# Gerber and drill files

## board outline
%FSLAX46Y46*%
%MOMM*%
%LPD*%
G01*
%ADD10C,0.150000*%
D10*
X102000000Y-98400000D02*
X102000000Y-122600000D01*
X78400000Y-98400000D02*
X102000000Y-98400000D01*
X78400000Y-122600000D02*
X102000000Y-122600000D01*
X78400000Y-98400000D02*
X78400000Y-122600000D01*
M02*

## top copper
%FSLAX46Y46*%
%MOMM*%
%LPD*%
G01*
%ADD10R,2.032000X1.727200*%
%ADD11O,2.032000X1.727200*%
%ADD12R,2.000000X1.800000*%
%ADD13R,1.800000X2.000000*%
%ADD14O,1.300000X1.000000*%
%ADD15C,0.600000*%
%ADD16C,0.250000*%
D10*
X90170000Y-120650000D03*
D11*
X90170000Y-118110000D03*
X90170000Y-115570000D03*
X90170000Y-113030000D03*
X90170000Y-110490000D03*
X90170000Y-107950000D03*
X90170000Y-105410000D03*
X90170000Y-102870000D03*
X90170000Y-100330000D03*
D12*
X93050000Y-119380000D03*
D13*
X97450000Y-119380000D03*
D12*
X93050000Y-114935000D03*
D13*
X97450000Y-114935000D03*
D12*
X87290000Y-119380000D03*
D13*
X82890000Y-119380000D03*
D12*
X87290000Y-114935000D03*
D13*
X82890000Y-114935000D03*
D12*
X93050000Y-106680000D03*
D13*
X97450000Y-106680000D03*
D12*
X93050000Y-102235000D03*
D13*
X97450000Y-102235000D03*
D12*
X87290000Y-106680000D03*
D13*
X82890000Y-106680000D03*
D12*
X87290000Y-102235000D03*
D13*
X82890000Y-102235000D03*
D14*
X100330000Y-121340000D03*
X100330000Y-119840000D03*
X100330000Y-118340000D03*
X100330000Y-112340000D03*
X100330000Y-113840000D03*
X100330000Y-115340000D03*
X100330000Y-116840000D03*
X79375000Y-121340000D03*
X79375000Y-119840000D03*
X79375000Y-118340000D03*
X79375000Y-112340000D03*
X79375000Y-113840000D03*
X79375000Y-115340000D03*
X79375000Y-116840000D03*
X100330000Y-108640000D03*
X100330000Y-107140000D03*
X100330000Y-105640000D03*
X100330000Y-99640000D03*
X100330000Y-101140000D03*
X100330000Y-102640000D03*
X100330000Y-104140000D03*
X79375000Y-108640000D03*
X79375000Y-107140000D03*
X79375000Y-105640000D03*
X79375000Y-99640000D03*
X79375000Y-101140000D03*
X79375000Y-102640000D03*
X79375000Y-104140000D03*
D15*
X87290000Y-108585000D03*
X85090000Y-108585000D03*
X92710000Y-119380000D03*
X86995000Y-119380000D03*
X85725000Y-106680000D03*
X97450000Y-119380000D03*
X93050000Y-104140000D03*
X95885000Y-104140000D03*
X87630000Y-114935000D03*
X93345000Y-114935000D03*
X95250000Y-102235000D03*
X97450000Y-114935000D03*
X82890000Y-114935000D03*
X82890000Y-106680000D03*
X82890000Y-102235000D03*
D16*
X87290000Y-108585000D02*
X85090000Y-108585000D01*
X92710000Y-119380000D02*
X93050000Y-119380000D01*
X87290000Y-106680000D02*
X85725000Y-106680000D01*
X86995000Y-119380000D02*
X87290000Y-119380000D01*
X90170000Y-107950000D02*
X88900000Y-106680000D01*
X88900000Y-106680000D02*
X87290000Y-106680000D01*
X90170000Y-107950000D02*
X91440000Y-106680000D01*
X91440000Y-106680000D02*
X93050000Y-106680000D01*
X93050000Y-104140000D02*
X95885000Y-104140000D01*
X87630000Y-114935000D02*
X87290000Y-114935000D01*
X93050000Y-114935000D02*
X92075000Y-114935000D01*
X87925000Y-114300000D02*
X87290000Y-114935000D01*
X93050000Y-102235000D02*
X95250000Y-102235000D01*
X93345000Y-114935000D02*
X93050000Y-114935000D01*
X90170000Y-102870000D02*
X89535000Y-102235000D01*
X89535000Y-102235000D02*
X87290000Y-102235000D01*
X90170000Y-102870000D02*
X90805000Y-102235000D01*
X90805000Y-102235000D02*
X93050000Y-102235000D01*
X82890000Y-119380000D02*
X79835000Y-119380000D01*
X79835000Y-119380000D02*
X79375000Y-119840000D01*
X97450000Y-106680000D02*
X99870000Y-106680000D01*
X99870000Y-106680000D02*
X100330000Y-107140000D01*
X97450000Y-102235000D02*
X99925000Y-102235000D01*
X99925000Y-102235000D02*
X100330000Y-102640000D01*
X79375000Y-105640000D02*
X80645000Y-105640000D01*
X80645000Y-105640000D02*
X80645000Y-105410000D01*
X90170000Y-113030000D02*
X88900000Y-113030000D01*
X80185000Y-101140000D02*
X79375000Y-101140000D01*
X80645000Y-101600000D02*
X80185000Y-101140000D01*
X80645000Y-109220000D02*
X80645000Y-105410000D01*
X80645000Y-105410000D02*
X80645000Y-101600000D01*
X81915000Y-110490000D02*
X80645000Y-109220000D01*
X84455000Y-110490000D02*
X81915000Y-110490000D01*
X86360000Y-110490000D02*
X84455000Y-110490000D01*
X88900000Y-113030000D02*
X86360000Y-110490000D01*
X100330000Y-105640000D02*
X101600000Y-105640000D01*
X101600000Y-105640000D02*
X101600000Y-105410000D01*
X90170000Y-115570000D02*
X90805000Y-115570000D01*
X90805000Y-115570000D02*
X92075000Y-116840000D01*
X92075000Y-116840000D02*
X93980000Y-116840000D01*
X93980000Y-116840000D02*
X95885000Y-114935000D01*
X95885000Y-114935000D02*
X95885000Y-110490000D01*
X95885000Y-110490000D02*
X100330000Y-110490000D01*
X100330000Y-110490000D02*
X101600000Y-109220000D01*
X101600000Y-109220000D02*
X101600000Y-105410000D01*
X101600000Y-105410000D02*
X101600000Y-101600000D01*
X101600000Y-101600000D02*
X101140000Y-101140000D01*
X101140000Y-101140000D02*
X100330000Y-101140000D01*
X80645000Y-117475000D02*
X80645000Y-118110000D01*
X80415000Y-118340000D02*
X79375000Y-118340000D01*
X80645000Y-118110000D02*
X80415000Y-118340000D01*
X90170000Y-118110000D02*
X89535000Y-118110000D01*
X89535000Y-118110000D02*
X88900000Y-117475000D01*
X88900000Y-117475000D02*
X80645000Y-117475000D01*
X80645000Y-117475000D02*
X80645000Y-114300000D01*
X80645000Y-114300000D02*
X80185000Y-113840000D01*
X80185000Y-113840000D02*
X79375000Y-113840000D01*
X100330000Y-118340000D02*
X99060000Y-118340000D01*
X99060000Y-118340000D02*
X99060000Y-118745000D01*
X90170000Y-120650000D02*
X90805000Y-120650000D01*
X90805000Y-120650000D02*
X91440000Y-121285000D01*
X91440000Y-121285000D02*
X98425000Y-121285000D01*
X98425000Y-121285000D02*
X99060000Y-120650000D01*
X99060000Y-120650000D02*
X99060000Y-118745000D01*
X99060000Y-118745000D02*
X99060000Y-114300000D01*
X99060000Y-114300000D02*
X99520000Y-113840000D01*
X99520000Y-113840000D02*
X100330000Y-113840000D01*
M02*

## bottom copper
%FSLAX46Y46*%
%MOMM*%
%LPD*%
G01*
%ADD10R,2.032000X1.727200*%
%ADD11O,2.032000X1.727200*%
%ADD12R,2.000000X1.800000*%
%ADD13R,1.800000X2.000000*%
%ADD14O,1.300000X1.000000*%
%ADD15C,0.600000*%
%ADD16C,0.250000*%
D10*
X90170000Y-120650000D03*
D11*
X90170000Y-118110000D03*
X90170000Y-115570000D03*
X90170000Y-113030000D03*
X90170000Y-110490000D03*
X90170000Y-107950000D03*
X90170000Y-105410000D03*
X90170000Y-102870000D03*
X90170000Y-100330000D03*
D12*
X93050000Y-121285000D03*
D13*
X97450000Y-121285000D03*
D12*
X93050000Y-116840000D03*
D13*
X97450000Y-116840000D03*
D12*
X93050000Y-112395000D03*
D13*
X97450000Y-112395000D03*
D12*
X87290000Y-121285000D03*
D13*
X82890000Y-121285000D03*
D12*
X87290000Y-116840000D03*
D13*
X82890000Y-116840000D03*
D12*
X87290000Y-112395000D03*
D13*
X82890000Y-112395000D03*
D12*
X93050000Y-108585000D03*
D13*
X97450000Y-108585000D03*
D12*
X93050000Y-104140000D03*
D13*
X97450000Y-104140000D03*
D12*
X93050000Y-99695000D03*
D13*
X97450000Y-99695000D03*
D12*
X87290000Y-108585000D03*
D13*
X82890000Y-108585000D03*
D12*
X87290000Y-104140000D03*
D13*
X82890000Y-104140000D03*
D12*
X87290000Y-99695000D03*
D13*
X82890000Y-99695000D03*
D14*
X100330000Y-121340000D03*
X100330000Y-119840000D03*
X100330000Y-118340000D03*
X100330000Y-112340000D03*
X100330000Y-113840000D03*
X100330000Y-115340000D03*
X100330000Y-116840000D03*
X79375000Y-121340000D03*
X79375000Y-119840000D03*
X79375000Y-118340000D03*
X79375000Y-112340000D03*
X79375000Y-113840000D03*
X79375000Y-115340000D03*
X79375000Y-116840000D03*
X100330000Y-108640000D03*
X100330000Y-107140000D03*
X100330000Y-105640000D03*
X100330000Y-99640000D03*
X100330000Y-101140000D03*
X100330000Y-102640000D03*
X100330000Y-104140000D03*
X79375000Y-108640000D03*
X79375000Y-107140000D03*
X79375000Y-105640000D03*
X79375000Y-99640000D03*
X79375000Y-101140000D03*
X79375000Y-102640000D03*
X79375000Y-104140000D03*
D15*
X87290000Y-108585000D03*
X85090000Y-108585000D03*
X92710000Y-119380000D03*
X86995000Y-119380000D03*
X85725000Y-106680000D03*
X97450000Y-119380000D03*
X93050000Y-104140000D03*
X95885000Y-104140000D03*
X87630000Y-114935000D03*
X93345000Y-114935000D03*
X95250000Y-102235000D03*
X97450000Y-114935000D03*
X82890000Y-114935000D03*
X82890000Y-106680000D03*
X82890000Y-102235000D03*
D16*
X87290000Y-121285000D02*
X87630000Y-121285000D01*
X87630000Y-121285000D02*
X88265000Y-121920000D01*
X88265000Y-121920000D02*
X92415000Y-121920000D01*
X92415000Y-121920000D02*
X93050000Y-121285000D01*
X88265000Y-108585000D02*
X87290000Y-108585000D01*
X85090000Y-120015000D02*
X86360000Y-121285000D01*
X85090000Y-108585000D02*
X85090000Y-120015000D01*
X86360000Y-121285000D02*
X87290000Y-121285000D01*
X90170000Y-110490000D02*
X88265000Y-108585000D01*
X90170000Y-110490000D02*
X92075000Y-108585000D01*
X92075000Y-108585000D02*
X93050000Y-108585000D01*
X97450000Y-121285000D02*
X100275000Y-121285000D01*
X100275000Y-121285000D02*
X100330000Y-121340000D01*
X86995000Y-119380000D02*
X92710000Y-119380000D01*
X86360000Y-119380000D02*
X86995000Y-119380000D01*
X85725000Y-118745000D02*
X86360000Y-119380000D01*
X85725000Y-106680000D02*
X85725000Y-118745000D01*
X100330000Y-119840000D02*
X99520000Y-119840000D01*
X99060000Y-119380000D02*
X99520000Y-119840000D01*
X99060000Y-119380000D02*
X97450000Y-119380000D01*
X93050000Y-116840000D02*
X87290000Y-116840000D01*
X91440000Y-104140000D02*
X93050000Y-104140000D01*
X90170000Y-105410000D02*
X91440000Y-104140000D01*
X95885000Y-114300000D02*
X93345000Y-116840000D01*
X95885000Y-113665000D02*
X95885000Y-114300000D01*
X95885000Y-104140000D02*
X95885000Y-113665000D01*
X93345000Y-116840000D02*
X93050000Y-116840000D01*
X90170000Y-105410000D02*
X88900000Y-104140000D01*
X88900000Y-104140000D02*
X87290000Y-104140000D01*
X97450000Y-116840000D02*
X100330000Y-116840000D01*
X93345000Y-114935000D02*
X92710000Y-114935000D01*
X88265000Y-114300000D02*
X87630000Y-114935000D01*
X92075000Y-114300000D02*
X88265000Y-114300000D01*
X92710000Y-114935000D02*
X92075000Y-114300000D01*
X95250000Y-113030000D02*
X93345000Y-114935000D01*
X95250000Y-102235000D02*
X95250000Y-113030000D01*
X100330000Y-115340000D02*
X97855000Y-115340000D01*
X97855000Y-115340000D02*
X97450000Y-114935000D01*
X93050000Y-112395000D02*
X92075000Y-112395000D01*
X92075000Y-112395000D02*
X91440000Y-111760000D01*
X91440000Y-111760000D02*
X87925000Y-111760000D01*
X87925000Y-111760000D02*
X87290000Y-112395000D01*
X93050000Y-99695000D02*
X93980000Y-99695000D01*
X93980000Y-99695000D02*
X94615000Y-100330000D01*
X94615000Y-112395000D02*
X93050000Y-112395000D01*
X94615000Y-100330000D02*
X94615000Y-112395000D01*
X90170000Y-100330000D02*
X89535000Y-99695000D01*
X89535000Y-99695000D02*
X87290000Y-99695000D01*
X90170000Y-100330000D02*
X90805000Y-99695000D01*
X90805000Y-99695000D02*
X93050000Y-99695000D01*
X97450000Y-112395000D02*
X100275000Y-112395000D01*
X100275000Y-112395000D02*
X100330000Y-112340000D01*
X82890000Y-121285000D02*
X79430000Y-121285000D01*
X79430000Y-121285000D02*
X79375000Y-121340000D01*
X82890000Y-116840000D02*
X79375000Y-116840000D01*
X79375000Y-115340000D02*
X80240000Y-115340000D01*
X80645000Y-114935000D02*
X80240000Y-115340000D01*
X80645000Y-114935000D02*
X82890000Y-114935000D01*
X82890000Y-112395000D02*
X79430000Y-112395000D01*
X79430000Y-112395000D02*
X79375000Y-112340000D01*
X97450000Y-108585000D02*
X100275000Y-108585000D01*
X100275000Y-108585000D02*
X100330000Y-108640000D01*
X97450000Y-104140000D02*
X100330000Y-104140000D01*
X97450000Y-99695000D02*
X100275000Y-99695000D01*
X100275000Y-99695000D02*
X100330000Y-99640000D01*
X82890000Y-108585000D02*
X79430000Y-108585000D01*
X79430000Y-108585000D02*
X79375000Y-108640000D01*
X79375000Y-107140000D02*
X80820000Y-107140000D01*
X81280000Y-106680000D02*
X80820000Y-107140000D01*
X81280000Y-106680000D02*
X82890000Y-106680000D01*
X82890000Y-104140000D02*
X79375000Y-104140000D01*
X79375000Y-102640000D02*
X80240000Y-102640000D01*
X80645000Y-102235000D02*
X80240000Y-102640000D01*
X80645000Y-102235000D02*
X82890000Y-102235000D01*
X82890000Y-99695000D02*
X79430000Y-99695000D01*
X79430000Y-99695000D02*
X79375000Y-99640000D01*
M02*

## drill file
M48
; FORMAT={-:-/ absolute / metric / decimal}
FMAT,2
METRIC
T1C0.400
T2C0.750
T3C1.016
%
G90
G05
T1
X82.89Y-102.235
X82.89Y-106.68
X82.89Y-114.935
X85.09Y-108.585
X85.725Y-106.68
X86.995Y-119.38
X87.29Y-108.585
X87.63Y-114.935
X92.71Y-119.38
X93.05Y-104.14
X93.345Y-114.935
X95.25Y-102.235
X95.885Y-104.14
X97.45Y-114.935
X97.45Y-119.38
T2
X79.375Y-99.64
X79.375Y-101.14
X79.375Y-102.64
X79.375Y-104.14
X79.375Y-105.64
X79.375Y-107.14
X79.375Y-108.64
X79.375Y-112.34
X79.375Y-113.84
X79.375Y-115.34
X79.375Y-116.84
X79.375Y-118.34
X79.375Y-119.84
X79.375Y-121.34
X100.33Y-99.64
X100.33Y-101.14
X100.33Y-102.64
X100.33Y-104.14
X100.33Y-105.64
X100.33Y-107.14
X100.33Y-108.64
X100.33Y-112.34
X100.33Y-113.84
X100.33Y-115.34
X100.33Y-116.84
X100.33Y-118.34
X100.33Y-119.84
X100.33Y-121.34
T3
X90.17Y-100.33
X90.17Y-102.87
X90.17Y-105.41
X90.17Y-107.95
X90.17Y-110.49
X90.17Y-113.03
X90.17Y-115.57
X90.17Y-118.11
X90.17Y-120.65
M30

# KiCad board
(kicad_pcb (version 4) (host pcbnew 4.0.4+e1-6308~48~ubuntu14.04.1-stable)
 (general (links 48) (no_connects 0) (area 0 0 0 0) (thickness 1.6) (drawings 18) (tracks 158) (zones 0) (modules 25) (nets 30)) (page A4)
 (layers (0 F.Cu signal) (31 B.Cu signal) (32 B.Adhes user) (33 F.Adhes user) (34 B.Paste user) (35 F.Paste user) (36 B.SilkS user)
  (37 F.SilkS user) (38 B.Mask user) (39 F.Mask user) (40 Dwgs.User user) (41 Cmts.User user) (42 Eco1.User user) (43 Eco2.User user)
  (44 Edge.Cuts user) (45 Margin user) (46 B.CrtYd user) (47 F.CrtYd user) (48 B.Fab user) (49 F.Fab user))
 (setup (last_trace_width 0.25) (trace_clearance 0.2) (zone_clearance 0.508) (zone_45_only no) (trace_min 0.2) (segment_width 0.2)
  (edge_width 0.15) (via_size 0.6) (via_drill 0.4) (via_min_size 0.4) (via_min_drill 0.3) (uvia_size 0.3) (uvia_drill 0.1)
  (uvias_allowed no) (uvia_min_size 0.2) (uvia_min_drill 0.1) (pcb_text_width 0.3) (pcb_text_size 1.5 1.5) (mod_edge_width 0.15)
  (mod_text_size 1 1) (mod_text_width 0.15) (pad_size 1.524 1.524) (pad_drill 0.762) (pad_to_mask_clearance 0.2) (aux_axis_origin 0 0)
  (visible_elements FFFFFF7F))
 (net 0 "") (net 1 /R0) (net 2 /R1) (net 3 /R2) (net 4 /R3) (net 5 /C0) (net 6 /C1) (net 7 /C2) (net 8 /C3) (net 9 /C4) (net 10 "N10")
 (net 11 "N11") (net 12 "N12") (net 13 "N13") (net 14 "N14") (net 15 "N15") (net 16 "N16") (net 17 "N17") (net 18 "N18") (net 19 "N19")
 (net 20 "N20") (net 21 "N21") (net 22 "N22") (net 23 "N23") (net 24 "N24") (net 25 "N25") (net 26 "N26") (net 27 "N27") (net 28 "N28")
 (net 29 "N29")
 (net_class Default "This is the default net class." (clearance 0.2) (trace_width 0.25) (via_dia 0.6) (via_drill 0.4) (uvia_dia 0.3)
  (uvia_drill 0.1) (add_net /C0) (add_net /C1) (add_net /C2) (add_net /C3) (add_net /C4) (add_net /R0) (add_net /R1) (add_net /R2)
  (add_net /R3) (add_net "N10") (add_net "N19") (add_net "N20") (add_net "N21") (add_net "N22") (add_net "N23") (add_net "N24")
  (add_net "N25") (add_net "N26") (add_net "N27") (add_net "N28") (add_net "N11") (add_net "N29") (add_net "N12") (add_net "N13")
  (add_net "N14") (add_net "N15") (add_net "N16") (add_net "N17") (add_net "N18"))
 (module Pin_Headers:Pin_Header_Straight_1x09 (layer B.Cu) (at 90.17 120.65)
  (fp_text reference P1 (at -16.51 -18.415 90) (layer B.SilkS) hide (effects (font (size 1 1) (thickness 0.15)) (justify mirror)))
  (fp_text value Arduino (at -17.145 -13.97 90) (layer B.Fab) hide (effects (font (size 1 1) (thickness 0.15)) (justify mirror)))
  (pad 1 thru_hole rect (at 0 0) (size 2.032 1.7272) (drill 1.016) (layers *.Cu *.Mask B.SilkS) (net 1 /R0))
  (pad 2 thru_hole oval (at 0 -2.54) (size 2.032 1.7272) (drill 1.016) (layers *.Cu *.Mask B.SilkS) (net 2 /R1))
  (pad 3 thru_hole oval (at 0 -5.08) (size 2.032 1.7272) (drill 1.016) (layers *.Cu *.Mask B.SilkS) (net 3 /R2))
  (pad 4 thru_hole oval (at 0 -7.62) (size 2.032 1.7272) (drill 1.016) (layers *.Cu *.Mask B.SilkS) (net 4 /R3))
  (pad 5 thru_hole oval (at 0 -10.16) (size 2.032 1.7272) (drill 1.016) (layers *.Cu *.Mask B.SilkS) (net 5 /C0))
  (pad 6 thru_hole oval (at 0 -12.7) (size 2.032 1.7272) (drill 1.016) (layers *.Cu *.Mask B.SilkS) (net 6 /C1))
  (pad 7 thru_hole oval (at 0 -15.24) (size 2.032 1.7272) (drill 1.016) (layers *.Cu *.Mask B.SilkS) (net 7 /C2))
  (pad 8 thru_hole oval (at 0 -17.78) (size 2.032 1.7272) (drill 1.016) (layers *.Cu *.Mask B.SilkS) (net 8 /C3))
  (pad 9 thru_hole oval (at 0 -20.32) (size 2.032 1.7272) (drill 1.016) (layers *.Cu *.Mask B.SilkS) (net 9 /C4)))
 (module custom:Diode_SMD (layer B.Cu) (at 95.25 121.285 180)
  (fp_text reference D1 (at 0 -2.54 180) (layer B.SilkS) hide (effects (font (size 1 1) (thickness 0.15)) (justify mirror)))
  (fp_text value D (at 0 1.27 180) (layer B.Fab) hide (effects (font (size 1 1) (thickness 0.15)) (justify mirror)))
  (pad 2 smd rect (at 2.2 0 180) (size 2 1.8) (layers B.Cu B.Paste B.Mask) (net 5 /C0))
  (pad 1 smd rect (at -2.2 0 180) (size 1.8 2) (layers B.Cu B.Paste B.Mask) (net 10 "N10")))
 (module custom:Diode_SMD (layer F.Cu) (at 95.25 119.38 180)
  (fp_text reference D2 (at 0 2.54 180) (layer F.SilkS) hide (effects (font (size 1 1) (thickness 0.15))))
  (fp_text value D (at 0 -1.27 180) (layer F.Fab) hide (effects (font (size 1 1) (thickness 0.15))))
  (pad 2 smd rect (at 2.2 0 180) (size 2 1.8) (layers F.Cu F.Paste F.Mask) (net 6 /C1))
  (pad 1 smd rect (at -2.2 0 180) (size 1.8 2) (layers F.Cu F.Paste F.Mask) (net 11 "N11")))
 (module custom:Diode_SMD (layer B.Cu) (at 95.25 116.84 180)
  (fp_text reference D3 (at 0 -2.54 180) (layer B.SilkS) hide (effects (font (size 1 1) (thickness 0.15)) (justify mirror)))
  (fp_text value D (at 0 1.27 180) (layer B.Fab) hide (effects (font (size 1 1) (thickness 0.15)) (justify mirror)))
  (pad 2 smd rect (at 2.2 0 180) (size 2 1.8) (layers B.Cu B.Paste B.Mask) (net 7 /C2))
  (pad 1 smd rect (at -2.2 0 180) (size 1.8 2) (layers B.Cu B.Paste B.Mask) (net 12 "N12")))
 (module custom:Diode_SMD (layer F.Cu) (at 95.25 114.935 180)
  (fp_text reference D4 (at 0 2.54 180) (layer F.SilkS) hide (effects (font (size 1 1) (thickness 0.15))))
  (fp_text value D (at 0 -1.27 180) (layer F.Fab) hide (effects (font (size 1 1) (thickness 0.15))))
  (pad 2 smd rect (at 2.2 0 180) (size 2 1.8) (layers F.Cu F.Paste F.Mask) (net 8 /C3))
  (pad 1 smd rect (at -2.2 0 180) (size 1.8 2) (layers F.Cu F.Paste F.Mask) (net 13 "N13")))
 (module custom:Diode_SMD (layer B.Cu) (at 95.25 112.395 180)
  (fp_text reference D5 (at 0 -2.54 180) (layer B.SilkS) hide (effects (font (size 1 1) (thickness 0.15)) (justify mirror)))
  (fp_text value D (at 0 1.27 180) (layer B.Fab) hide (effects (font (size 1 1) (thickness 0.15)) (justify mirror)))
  (pad 2 smd rect (at 2.2 0 180) (size 2 1.8) (layers B.Cu B.Paste B.Mask) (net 9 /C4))
  (pad 1 smd rect (at -2.2 0 180) (size 1.8 2) (layers B.Cu B.Paste B.Mask) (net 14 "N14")))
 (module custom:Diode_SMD (layer B.Cu) (at 85.09 121.285)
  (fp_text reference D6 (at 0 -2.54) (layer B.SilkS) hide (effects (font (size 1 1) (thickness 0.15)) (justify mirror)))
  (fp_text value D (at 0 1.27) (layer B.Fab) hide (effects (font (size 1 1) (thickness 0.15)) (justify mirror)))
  (pad 2 smd rect (at 2.2 0) (size 2 1.8) (layers B.Cu B.Paste B.Mask) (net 5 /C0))
  (pad 1 smd rect (at -2.2 0) (size 1.8 2) (layers B.Cu B.Paste B.Mask) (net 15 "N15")))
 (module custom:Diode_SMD (layer F.Cu) (at 85.09 119.38)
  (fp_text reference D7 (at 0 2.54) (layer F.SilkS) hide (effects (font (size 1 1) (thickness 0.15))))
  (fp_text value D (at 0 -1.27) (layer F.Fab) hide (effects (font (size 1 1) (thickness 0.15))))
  (pad 2 smd rect (at 2.2 0) (size 2 1.8) (layers F.Cu F.Paste F.Mask) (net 6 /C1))
  (pad 1 smd rect (at -2.2 0) (size 1.8 2) (layers F.Cu F.Paste F.Mask) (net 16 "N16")))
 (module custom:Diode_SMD (layer B.Cu) (at 85.09 116.84)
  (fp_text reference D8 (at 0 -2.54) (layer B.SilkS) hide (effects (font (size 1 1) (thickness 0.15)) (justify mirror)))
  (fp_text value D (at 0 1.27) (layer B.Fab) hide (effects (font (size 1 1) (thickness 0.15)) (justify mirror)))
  (pad 2 smd rect (at 2.2 0) (size 2 1.8) (layers B.Cu B.Paste B.Mask) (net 7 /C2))
  (pad 1 smd rect (at -2.2 0) (size 1.8 2) (layers B.Cu B.Paste B.Mask) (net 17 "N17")))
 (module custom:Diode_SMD (layer F.Cu) (at 85.09 114.935)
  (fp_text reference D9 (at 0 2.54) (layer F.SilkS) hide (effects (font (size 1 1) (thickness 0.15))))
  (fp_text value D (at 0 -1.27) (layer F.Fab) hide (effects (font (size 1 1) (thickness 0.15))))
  (pad 2 smd rect (at 2.2 0) (size 2 1.8) (layers F.Cu F.Paste F.Mask) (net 8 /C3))
  (pad 1 smd rect (at -2.2 0) (size 1.8 2) (layers F.Cu F.Paste F.Mask) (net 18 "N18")))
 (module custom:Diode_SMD (layer B.Cu) (at 85.09 112.395)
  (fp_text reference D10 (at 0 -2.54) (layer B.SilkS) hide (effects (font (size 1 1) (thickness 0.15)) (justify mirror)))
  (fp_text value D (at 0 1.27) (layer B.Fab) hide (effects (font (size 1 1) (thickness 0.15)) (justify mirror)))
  (pad 2 smd rect (at 2.2 0) (size 2 1.8) (layers B.Cu B.Paste B.Mask) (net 9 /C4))
  (pad 1 smd rect (at -2.2 0) (size 1.8 2) (layers B.Cu B.Paste B.Mask) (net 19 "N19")))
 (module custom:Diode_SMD (layer B.Cu) (at 95.25 108.585 180)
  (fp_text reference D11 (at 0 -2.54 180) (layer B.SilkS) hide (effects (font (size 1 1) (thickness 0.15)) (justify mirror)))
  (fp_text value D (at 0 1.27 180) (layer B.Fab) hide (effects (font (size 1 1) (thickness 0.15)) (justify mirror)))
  (pad 2 smd rect (at 2.2 0 180) (size 2 1.8) (layers B.Cu B.Paste B.Mask) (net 5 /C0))
  (pad 1 smd rect (at -2.2 0 180) (size 1.8 2) (layers B.Cu B.Paste B.Mask) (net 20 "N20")))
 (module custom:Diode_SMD (layer F.Cu) (at 95.25 106.68 180)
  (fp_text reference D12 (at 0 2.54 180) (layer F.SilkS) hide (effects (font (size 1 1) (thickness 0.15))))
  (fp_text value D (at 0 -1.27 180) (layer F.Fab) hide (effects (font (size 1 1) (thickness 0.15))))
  (pad 2 smd rect (at 2.2 0 180) (size 2 1.8) (layers F.Cu F.Paste F.Mask) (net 6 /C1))
  (pad 1 smd rect (at -2.2 0 180) (size 1.8 2) (layers F.Cu F.Paste F.Mask) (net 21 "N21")))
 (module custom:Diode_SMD (layer B.Cu) (at 95.25 104.14 180)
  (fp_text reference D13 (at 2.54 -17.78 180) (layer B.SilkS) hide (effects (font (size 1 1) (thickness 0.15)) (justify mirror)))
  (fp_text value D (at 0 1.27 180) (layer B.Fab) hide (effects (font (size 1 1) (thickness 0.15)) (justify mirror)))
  (pad 2 smd rect (at 2.2 0 180) (size 2 1.8) (layers B.Cu B.Paste B.Mask) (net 7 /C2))
  (pad 1 smd rect (at -2.2 0 180) (size 1.8 2) (layers B.Cu B.Paste B.Mask) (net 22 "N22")))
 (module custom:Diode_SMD (layer F.Cu) (at 95.25 102.235 180)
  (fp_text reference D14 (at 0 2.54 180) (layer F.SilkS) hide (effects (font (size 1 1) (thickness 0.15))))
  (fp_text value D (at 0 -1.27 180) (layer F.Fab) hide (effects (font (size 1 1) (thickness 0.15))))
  (pad 2 smd rect (at 2.2 0 180) (size 2 1.8) (layers F.Cu F.Paste F.Mask) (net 8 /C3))
  (pad 1 smd rect (at -2.2 0 180) (size 1.8 2) (layers F.Cu F.Paste F.Mask) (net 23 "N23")))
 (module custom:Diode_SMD (layer B.Cu) (at 95.25 99.695 180)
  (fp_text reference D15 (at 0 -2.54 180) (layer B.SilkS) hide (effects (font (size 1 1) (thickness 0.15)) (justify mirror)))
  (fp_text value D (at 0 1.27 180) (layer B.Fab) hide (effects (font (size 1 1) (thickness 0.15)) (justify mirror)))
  (pad 2 smd rect (at 2.2 0 180) (size 2 1.8) (layers B.Cu B.Paste B.Mask) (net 9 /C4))
  (pad 1 smd rect (at -2.2 0 180) (size 1.8 2) (layers B.Cu B.Paste B.Mask) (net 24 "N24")))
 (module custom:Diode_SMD (layer B.Cu) (at 85.09 108.585)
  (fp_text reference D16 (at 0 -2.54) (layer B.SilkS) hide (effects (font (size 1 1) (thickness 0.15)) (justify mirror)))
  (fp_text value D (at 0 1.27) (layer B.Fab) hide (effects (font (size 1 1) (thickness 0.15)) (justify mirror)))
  (pad 2 smd rect (at 2.2 0) (size 2 1.8) (layers B.Cu B.Paste B.Mask) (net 5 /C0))
  (pad 1 smd rect (at -2.2 0) (size 1.8 2) (layers B.Cu B.Paste B.Mask) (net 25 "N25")))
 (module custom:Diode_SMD (layer F.Cu) (at 85.09 106.68)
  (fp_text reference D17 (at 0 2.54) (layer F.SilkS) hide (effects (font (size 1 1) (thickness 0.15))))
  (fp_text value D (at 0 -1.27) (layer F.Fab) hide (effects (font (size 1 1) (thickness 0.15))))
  (pad 2 smd rect (at 2.2 0) (size 2 1.8) (layers F.Cu F.Paste F.Mask) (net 6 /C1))
  (pad 1 smd rect (at -2.2 0) (size 1.8 2) (layers F.Cu F.Paste F.Mask) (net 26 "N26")))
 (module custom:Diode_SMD (layer B.Cu) (at 85.09 104.14)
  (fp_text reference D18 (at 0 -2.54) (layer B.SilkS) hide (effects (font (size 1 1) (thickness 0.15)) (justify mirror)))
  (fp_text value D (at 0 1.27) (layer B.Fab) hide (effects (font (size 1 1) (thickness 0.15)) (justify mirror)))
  (pad 2 smd rect (at 2.2 0) (size 2 1.8) (layers B.Cu B.Paste B.Mask) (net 7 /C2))
  (pad 1 smd rect (at -2.2 0) (size 1.8 2) (layers B.Cu B.Paste B.Mask) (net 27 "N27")))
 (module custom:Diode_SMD (layer F.Cu) (at 85.09 102.235)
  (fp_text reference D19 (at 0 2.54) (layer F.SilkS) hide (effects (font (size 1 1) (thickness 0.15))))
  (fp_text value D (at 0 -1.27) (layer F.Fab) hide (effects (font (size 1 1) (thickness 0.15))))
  (pad 2 smd rect (at 2.2 0) (size 2 1.8) (layers F.Cu F.Paste F.Mask) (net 8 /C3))
  (pad 1 smd rect (at -2.2 0) (size 1.8 2) (layers F.Cu F.Paste F.Mask) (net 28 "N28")))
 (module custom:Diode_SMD (layer B.Cu) (at 85.09 99.695)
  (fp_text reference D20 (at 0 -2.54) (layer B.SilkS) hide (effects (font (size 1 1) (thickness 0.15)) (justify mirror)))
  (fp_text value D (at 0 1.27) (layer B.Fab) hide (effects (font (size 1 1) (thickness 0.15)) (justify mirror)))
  (pad 2 smd rect (at 2.2 0) (size 2 1.8) (layers B.Cu B.Paste B.Mask) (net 9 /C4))
  (pad 1 smd rect (at -2.2 0) (size 1.8 2) (layers B.Cu B.Paste B.Mask) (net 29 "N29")))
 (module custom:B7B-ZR (layer F.Cu) (at 100.33 116.84 90)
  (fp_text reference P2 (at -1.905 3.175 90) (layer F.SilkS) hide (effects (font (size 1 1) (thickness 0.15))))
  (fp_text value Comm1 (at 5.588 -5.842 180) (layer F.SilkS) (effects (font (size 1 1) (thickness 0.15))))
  (pad 1 thru_hole oval (at -4.5 0 90) (size 1 1.3) (drill 0.75) (layers *.Cu *.Mask F.Paste) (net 10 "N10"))
  (pad 2 thru_hole oval (at -3 0 90) (size 1 1.3) (drill 0.75) (layers *.Cu *.Mask F.Paste) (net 11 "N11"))
  (pad 3 thru_hole oval (at -1.5 0 90) (size 1 1.3) (drill 0.75) (layers *.Cu *.Mask F.Paste) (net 1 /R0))
  (pad 7 thru_hole oval (at 4.5 0 90) (size 1 1.3) (drill 0.75) (layers *.Cu *.Mask F.Paste) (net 14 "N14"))
  (pad 6 thru_hole oval (at 3 0 90) (size 1 1.3) (drill 0.75) (layers *.Cu *.Mask F.Paste) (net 1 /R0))
  (pad 5 thru_hole oval (at 1.5 0 90) (size 1 1.3) (drill 0.75) (layers *.Cu *.Mask F.Paste) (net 13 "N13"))
  (pad 4 thru_hole oval (at 0 0 90) (size 1 1.3) (drill 0.75) (layers *.Cu *.Mask F.Paste) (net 12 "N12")))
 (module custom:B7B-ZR (layer F.Cu) (at 79.375 116.84 90)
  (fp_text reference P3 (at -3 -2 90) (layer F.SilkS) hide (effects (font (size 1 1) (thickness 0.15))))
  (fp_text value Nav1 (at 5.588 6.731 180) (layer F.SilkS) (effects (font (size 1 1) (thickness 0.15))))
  (pad 1 thru_hole oval (at -4.5 0 90) (size 1 1.3) (drill 0.75) (layers *.Cu *.Mask F.Paste) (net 15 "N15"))
  (pad 2 thru_hole oval (at -3 0 90) (size 1 1.3) (drill 0.75) (layers *.Cu *.Mask F.Paste) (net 16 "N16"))
  (pad 3 thru_hole oval (at -1.5 0 90) (size 1 1.3) (drill 0.75) (layers *.Cu *.Mask F.Paste) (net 2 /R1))
  (pad 7 thru_hole oval (at 4.5 0 90) (size 1 1.3) (drill 0.75) (layers *.Cu *.Mask F.Paste) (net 19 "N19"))
  (pad 6 thru_hole oval (at 3 0 90) (size 1 1.3) (drill 0.75) (layers *.Cu *.Mask F.Paste) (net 2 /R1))
  (pad 5 thru_hole oval (at 1.5 0 90) (size 1 1.3) (drill 0.75) (layers *.Cu *.Mask F.Paste) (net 18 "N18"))
  (pad 4 thru_hole oval (at 0 0 90) (size 1 1.3) (drill 0.75) (layers *.Cu *.Mask F.Paste) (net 17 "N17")))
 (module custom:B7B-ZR (layer F.Cu) (at 100.33 104.14 90)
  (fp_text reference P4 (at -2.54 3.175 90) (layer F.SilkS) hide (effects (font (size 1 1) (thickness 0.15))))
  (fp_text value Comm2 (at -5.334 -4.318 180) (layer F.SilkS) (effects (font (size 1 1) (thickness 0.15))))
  (pad 1 thru_hole oval (at -4.5 0 90) (size 1 1.3) (drill 0.75) (layers *.Cu *.Mask F.Paste) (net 20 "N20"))
  (pad 2 thru_hole oval (at -3 0 90) (size 1 1.3) (drill 0.75) (layers *.Cu *.Mask F.Paste) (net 21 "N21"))
  (pad 3 thru_hole oval (at -1.5 0 90) (size 1 1.3) (drill 0.75) (layers *.Cu *.Mask F.Paste) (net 3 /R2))
  (pad 7 thru_hole oval (at 4.5 0 90) (size 1 1.3) (drill 0.75) (layers *.Cu *.Mask F.Paste) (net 24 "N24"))
  (pad 6 thru_hole oval (at 3 0 90) (size 1 1.3) (drill 0.75) (layers *.Cu *.Mask F.Paste) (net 3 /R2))
  (pad 5 thru_hole oval (at 1.5 0 90) (size 1 1.3) (drill 0.75) (layers *.Cu *.Mask F.Paste) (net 23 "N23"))
  (pad 4 thru_hole oval (at 0 0 90) (size 1 1.3) (drill 0.75) (layers *.Cu *.Mask F.Paste) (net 22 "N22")))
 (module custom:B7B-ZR (layer F.Cu) (at 79.375 104.14 90)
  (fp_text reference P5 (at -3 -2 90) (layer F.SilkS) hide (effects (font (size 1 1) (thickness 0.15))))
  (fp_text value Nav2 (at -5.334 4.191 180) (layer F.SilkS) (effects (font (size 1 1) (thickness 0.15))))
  (pad 1 thru_hole oval (at -4.5 0 90) (size 1 1.3) (drill 0.75) (layers *.Cu *.Mask F.Paste) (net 25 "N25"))
  (pad 2 thru_hole oval (at -3 0 90) (size 1 1.3) (drill 0.75) (layers *.Cu *.Mask F.Paste) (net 26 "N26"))
  (pad 3 thru_hole oval (at -1.5 0 90) (size 1 1.3) (drill 0.75) (layers *.Cu *.Mask F.Paste) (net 4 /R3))
  (pad 7 thru_hole oval (at 4.5 0 90) (size 1 1.3) (drill 0.75) (layers *.Cu *.Mask F.Paste) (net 29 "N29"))
  (pad 6 thru_hole oval (at 3 0 90) (size 1 1.3) (drill 0.75) (layers *.Cu *.Mask F.Paste) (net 4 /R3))
  (pad 5 thru_hole oval (at 1.5 0 90) (size 1 1.3) (drill 0.75) (layers *.Cu *.Mask F.Paste) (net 28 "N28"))
  (pad 4 thru_hole oval (at 0 0 90) (size 1 1.3) (drill 0.75) (layers *.Cu *.Mask F.Paste) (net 27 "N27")))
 (gr_line (start 102 98.4) (end 102 122.6) (angle 90) (layer Edge.Cuts) (width 0.15))
 (gr_line (start 78.4 98.4) (end 102 98.4) (angle 90) (layer Edge.Cuts) (width 0.15))
 (gr_line (start 78.4 122.6) (end 102 122.6) (angle 90) (layer Edge.Cuts) (width 0.15))
 (gr_line (start 78.4 98.4) (end 78.4 122.6) (angle 90) (layer Edge.Cuts) (width 0.15))
 (segment (start 87.29 121.285) (end 87.63 121.285) (width 0.25) (layer B.Cu) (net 5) (status C00000))
 (segment (start 87.63 121.285) (end 88.265 121.92) (width 0.25) (layer B.Cu) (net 5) (status C00000))
 (segment (start 88.265 121.92) (end 92.415 121.92) (width 0.25) (layer B.Cu) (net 5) (status C00000))
 (segment (start 92.415 121.92) (end 93.05 121.285) (width 0.25) (layer B.Cu) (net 5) (status C00000))
 (via (at 87.29 108.585) (size 0.6) (drill 0.4) (layers F.Cu B.Cu) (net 5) (status 400000))
 (segment (start 88.265 108.585) (end 87.29 108.585) (width 0.25) (layer B.Cu) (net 5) (status C00000))
 (segment (start 85.09 120.015) (end 86.36 121.285) (width 0.25) (layer B.Cu) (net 5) (status 800000))
 (segment (start 85.09 108.585) (end 85.09 120.015) (width 0.25) (layer B.Cu) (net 5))
 (via (at 85.09 108.585) (size 0.6) (drill 0.4) (layers F.Cu B.Cu) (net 5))
 (segment (start 87.29 108.585) (end 85.09 108.585) (width 0.25) (layer F.Cu) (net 5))
 (segment (start 86.36 121.285) (end 87.29 121.285) (width 0.25) (layer B.Cu) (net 5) (status C00000))
 (segment (start 90.17 110.49) (end 88.265 108.585) (width 0.25) (layer B.Cu) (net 5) (status C00000))
 (segment (start 90.17 110.49) (end 92.075 108.585) (width 0.25) (layer B.Cu) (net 5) (status C00000))
 (segment (start 92.075 108.585) (end 93.05 108.585) (width 0.25) (layer B.Cu) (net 5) (status C00000))
 (segment (start 97.45 121.285) (end 100.275 121.285) (width 0.25) (layer B.Cu) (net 10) (status C00000))
 (segment (start 100.275 121.285) (end 100.33 121.34) (width 0.25) (layer B.Cu) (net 10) (status C00000))
 (segment (start 86.995 119.38) (end 92.71 119.38) (width 0.25) (layer B.Cu) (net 6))
 (segment (start 92.71 119.38) (end 93.05 119.38) (width 0.25) (layer F.Cu) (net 6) (status C00000))
 (via (at 92.71 119.38) (size 0.6) (drill 0.4) (layers F.Cu B.Cu) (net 6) (status 800000))
 (segment (start 87.29 106.68) (end 85.725 106.68) (width 0.25) (layer F.Cu) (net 6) (status 400000))
 (segment (start 86.995 119.38) (end 87.29 119.38) (width 0.25) (layer F.Cu) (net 6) (status C00000))
 (via (at 86.995 119.38) (size 0.6) (drill 0.4) (layers F.Cu B.Cu) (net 6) (status 800000))
 (segment (start 86.36 119.38) (end 86.995 119.38) (width 0.25) (layer B.Cu) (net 6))
 (segment (start 85.725 118.745) (end 86.36 119.38) (width 0.25) (layer B.Cu) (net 6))
 (segment (start 85.725 106.68) (end 85.725 118.745) (width 0.25) (layer B.Cu) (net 6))
 (via (at 85.725 106.68) (size 0.6) (drill 0.4) (layers F.Cu B.Cu) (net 6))
 (segment (start 90.17 107.95) (end 88.9 106.68) (width 0.25) (layer F.Cu) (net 6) (status 400000))
 (segment (start 88.9 106.68) (end 87.29 106.68) (width 0.25) (layer F.Cu) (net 6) (status 800000))
 (segment (start 90.17 107.95) (end 91.44 106.68) (width 0.25) (layer F.Cu) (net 6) (status 400000))
 (segment (start 91.44 106.68) (end 93.05 106.68) (width 0.25) (layer F.Cu) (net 6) (status 800000))
 (via (at 97.45 119.38) (size 0.6) (drill 0.4) (layers F.Cu B.Cu) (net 11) (status C00000))
 (segment (start 100.33 119.84) (end 99.52 119.84) (width 0.25) (layer B.Cu) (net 11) (status 400000))
 (segment (start 99.06 119.38) (end 99.52 119.84) (width 0.25) (layer B.Cu) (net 11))
 (segment (start 99.06 119.38) (end 97.45 119.38) (width 0.25) (layer B.Cu) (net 11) (status 800000))
 (segment (start 93.05 116.84) (end 87.29 116.84) (width 0.25) (layer B.Cu) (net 7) (status C00000))
 (via (at 93.05 104.14) (size 0.6) (drill 0.4) (layers F.Cu B.Cu) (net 7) (status 400000))
 (segment (start 91.44 104.14) (end 93.05 104.14) (width 0.25) (layer B.Cu) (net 7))
 (segment (start 90.17 105.41) (end 91.44 104.14) (width 0.25) (layer B.Cu) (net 7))
 (segment (start 95.885 114.3) (end 93.345 116.84) (width 0.25) (layer B.Cu) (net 7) (status 800000))
 (segment (start 95.885 113.665) (end 95.885 114.3) (width 0.25) (layer B.Cu) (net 7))
 (segment (start 95.885 104.14) (end 95.885 113.665) (width 0.25) (layer B.Cu) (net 7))
 (via (at 95.885 104.14) (size 0.6) (drill 0.4) (layers F.Cu B.Cu) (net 7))
 (segment (start 93.05 104.14) (end 95.885 104.14) (width 0.25) (layer F.Cu) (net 7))
 (segment (start 93.345 116.84) (end 93.05 116.84) (width 0.25) (layer B.Cu) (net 7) (status C00000))
 (segment (start 90.17 105.41) (end 88.9 104.14) (width 0.25) (layer B.Cu) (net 7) (status 400000))
 (segment (start 88.9 104.14) (end 87.29 104.14) (width 0.25) (layer B.Cu) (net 7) (status 800000))
 (segment (start 97.45 116.84) (end 100.33 116.84) (width 0.25) (layer B.Cu) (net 12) (status C00000))
 (segment (start 93.345 114.935) (end 92.71 114.935) (width 0.25) (layer B.Cu) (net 8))
 (segment (start 87.63 114.935) (end 87.29 114.935) (width 0.25) (layer F.Cu) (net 8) (status C00000))
 (via (at 87.63 114.935) (size 0.6) (drill 0.4) (layers F.Cu B.Cu) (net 8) (status 800000))
 (segment (start 88.265 114.3) (end 87.63 114.935) (width 0.25) (layer B.Cu) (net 8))
 (segment (start 92.075 114.3) (end 88.265 114.3) (width 0.25) (layer B.Cu) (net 8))
 (segment (start 92.71 114.935) (end 92.075 114.3) (width 0.25) (layer B.Cu) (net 8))
 (segment (start 93.05 114.935) (end 92.075 114.935) (width 0.25) (layer F.Cu) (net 8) (status C00000))
 (segment (start 87.925 114.3) (end 87.29 114.935) (width 0.25) (layer F.Cu) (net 8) (status C00000))
 (segment (start 93.05 102.235) (end 95.25 102.235) (width 0.25) (layer F.Cu) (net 8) (status 400000))
 (segment (start 93.345 114.935) (end 93.05 114.935) (width 0.25) (layer F.Cu) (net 8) (status C00000))
 (via (at 93.345 114.935) (size 0.6) (drill 0.4) (layers F.Cu B.Cu) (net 8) (status 800000))
 (segment (start 95.25 113.03) (end 93.345 114.935) (width 0.25) (layer B.Cu) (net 8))
 (segment (start 95.25 102.235) (end 95.25 113.03) (width 0.25) (layer B.Cu) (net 8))
 (via (at 95.25 102.235) (size 0.6) (drill 0.4) (layers F.Cu B.Cu) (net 8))
 (segment (start 90.17 102.87) (end 89.535 102.235) (width 0.25) (layer F.Cu) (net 8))
 (segment (start 89.535 102.235) (end 87.29 102.235) (width 0.25) (layer F.Cu) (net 8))
 (segment (start 90.17 102.87) (end 90.805 102.235) (width 0.25) (layer F.Cu) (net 8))
 (segment (start 90.805 102.235) (end 93.05 102.235) (width 0.25) (layer F.Cu) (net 8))
 (via (at 97.45 114.935) (size 0.6) (drill 0.4) (layers F.Cu B.Cu) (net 13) (status C00000))
 (segment (start 100.33 115.34) (end 97.855 115.34) (width 0.25) (layer B.Cu) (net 13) (status 400000))
 (segment (start 97.855 115.34) (end 97.45 114.935) (width 0.25) (layer B.Cu) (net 13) (status 800000))
 (segment (start 93.05 112.395) (end 92.075 112.395) (width 0.25) (layer B.Cu) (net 9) (status C00000))
 (segment (start 92.075 112.395) (end 91.44 111.76) (width 0.25) (layer B.Cu) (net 9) (status 400000))
 (segment (start 91.44 111.76) (end 87.925 111.76) (width 0.25) (layer B.Cu) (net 9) (status 800000))
 (segment (start 87.925 111.76) (end 87.29 112.395) (width 0.25) (layer B.Cu) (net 9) (status C00000))
 (segment (start 93.05 99.695) (end 93.98 99.695) (width 0.25) (layer B.Cu) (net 9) (status C00000))
 (segment (start 93.98 99.695) (end 94.615 100.33) (width 0.25) (layer B.Cu) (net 9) (status 400000))
 (segment (start 94.615 112.395) (end 93.05 112.395) (width 0.25) (layer B.Cu) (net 9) (status 800000))
 (segment (start 94.615 100.33) (end 94.615 112.395) (width 0.25) (layer B.Cu) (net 9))
 (segment (start 90.17 100.33) (end 89.535 99.695) (width 0.25) (layer B.Cu) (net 9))
 (segment (start 89.535 99.695) (end 87.29 99.695) (width 0.25) (layer B.Cu) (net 9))
 (segment (start 90.17 100.33) (end 90.805 99.695) (width 0.25) (layer B.Cu) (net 9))
 (segment (start 90.805 99.695) (end 93.05 99.695) (width 0.25) (layer B.Cu) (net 9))
 (segment (start 97.45 112.395) (end 100.275 112.395) (width 0.25) (layer B.Cu) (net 14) (status C00000))
 (segment (start 100.275 112.395) (end 100.33 112.34) (width 0.25) (layer B.Cu) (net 14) (status C00000))
 (segment (start 82.89 121.285) (end 79.43 121.285) (width 0.25) (layer B.Cu) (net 15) (status C00000))
 (segment (start 79.43 121.285) (end 79.375 121.34) (width 0.25) (layer B.Cu) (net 15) (status C00000))
 (segment (start 82.89 119.38) (end 79.835 119.38) (width 0.25) (layer F.Cu) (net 16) (status 400000))
 (segment (start 79.835 119.38) (end 79.375 119.84) (width 0.25) (layer F.Cu) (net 16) (status 800000))
 (segment (start 82.89 116.84) (end 79.375 116.84) (width 0.25) (layer B.Cu) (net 17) (status C00000))
 (via (at 82.89 114.935) (size 0.6) (drill 0.4) (layers F.Cu B.Cu) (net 18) (status C00000))
 (segment (start 79.375 115.34) (end 80.24 115.34) (width 0.25) (layer B.Cu) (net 18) (status 400000))
 (segment (start 80.645 114.935) (end 80.24 115.34) (width 0.25) (layer B.Cu) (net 18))
 (segment (start 80.645 114.935) (end 82.89 114.935) (width 0.25) (layer B.Cu) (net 18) (status 800000))
 (segment (start 82.89 112.395) (end 79.43 112.395) (width 0.25) (layer B.Cu) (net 19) (status C00000))
 (segment (start 79.43 112.395) (end 79.375 112.34) (width 0.25) (layer B.Cu) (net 19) (status C00000))
 (segment (start 97.45 108.585) (end 100.275 108.585) (width 0.25) (layer B.Cu) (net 20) (status C00000))
 (segment (start 100.275 108.585) (end 100.33 108.64) (width 0.25) (layer B.Cu) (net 20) (status C00000))
 (segment (start 97.45 106.68) (end 99.87 106.68) (width 0.25) (layer F.Cu) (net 21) (status 400000))
 (segment (start 99.87 106.68) (end 100.33 107.14) (width 0.25) (layer F.Cu) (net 21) (status 800000))
 (segment (start 97.45 104.14) (end 100.33 104.14) (width 0.25) (layer B.Cu) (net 22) (status C00000))
 (segment (start 97.45 102.235) (end 99.925 102.235) (width 0.25) (layer F.Cu) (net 23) (status C00000))
 (segment (start 99.925 102.235) (end 100.33 102.64) (width 0.25) (layer F.Cu) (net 23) (status C00000))
 (segment (start 97.45 99.695) (end 100.275 99.695) (width 0.25) (layer B.Cu) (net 24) (status C00000))
 (segment (start 100.275 99.695) (end 100.33 99.64) (width 0.25) (layer B.Cu) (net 24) (status C00000))
 (segment (start 82.89 108.585) (end 79.43 108.585) (width 0.25) (layer B.Cu) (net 25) (status C00000))
 (segment (start 79.43 108.585) (end 79.375 108.64) (width 0.25) (layer B.Cu) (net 25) (status C00000))
 (via (at 82.89 106.68) (size 0.6) (drill 0.4) (layers F.Cu B.Cu) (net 26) (status C00000))
 (segment (start 79.375 107.14) (end 80.82 107.14) (width 0.25) (layer B.Cu) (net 26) (status 400000))
 (segment (start 81.28 106.68) (end 80.82 107.14) (width 0.25) (layer B.Cu) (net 26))
 (segment (start 81.28 106.68) (end 82.89 106.68) (width 0.25) (layer B.Cu) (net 26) (status 800000))
 (segment (start 82.89 104.14) (end 79.375 104.14) (width 0.25) (layer B.Cu) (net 27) (status C00000))
 (via (at 82.89 102.235) (size 0.6) (drill 0.4) (layers F.Cu B.Cu) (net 28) (status C00000))
 (segment (start 79.375 102.64) (end 80.24 102.64) (width 0.25) (layer B.Cu) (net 28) (status 400000))
 (segment (start 80.645 102.235) (end 80.24 102.64) (width 0.25) (layer B.Cu) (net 28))
 (segment (start 80.645 102.235) (end 82.89 102.235) (width 0.25) (layer B.Cu) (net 28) (status 800000))
 (segment (start 82.89 99.695) (end 79.43 99.695) (width 0.25) (layer B.Cu) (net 29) (status C00000))
 (segment (start 79.43 99.695) (end 79.375 99.64) (width 0.25) (layer B.Cu) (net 29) (status C00000))
 (segment (start 79.375 105.64) (end 80.645 105.64) (width 0.25) (layer F.Cu) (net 4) (status 400000))
 (segment (start 80.645 105.64) (end 80.645 105.41) (width 0.25) (layer F.Cu) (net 4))
 (segment (start 90.17 113.03) (end 88.9 113.03) (width 0.25) (layer F.Cu) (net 4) (status 400000))
 (segment (start 80.185 101.14) (end 79.375 101.14) (width 0.25) (layer F.Cu) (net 4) (status 800000))
 (segment (start 80.645 101.6) (end 80.185 101.14) (width 0.25) (layer F.Cu) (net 4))
 (segment (start 80.645 109.22) (end 80.645 105.41) (width 0.25) (layer F.Cu) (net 4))
 (segment (start 80.645 105.41) (end 80.645 101.6) (width 0.25) (layer F.Cu) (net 4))
 (segment (start 81.915 110.49) (end 80.645 109.22) (width 0.25) (layer F.Cu) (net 4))
 (segment (start 84.455 110.49) (end 81.915 110.49) (width 0.25) (layer F.Cu) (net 4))
 (segment (start 86.36 110.49) (end 84.455 110.49) (width 0.25) (layer F.Cu) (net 4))
 (segment (start 88.9 113.03) (end 86.36 110.49) (width 0.25) (layer F.Cu) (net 4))
 (segment (start 100.33 105.64) (end 101.6 105.64) (width 0.25) (layer F.Cu) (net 3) (status 400000))
 (segment (start 101.6 105.64) (end 101.6 105.41) (width 0.25) (layer F.Cu) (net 3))
 (segment (start 90.17 115.57) (end 90.805 115.57) (width 0.25) (layer F.Cu) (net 3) (status C00000))
 (segment (start 90.805 115.57) (end 92.075 116.84) (width 0.25) (layer F.Cu) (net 3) (status 400000))
 (segment (start 92.075 116.84) (end 93.98 116.84) (width 0.25) (layer F.Cu) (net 3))
 (segment (start 93.98 116.84) (end 95.885 114.935) (width 0.25) (layer F.Cu) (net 3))
 (segment (start 95.885 114.935) (end 95.885 110.49) (width 0.25) (layer F.Cu) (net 3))
 (segment (start 95.885 110.49) (end 100.33 110.49) (width 0.25) (layer F.Cu) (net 3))
 (segment (start 100.33 110.49) (end 101.6 109.22) (width 0.25) (layer F.Cu) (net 3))
 (segment (start 101.6 109.22) (end 101.6 105.41) (width 0.25) (layer F.Cu) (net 3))
 (segment (start 101.6 105.41) (end 101.6 101.6) (width 0.25) (layer F.Cu) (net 3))
 (segment (start 101.6 101.6) (end 101.14 101.14) (width 0.25) (layer F.Cu) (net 3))
 (segment (start 101.14 101.14) (end 100.33 101.14) (width 0.25) (layer F.Cu) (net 3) (status 800000))
 (segment (start 80.645 117.475) (end 80.645 118.11) (width 0.25) (layer F.Cu) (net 2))
 (segment (start 80.415 118.34) (end 79.375 118.34) (width 0.25) (layer F.Cu) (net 2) (status 800000))
 (segment (start 80.645 118.11) (end 80.415 118.34) (width 0.25) (layer F.Cu) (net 2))
 (segment (start 90.17 118.11) (end 89.535 118.11) (width 0.25) (layer F.Cu) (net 2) (status C00000))
 (segment (start 89.535 118.11) (end 88.9 117.475) (width 0.25) (layer F.Cu) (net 2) (status 400000))
 (segment (start 88.9 117.475) (end 80.645 117.475) (width 0.25) (layer F.Cu) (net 2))
 (segment (start 80.645 117.475) (end 80.645 114.3) (width 0.25) (layer F.Cu) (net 2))
 (segment (start 80.645 114.3) (end 80.185 113.84) (width 0.25) (layer F.Cu) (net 2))
 (segment (start 80.185 113.84) (end 79.375 113.84) (width 0.25) (layer F.Cu) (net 2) (status 800000))
 (segment (start 100.33 118.34) (end 99.06 118.34) (width 0.25) (layer F.Cu) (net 1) (status 400000))
 (segment (start 99.06 118.34) (end 99.06 118.745) (width 0.25) (layer F.Cu) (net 1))
 (segment (start 90.17 120.65) (end 90.805 120.65) (width 0.25) (layer F.Cu) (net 1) (status C00000))
 (segment (start 90.805 120.65) (end 91.44 121.285) (width 0.25) (layer F.Cu) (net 1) (status 400000))
 (segment (start 91.44 121.285) (end 98.425 121.285) (width 0.25) (layer F.Cu) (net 1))
 (segment (start 98.425 121.285) (end 99.06 120.65) (width 0.25) (layer F.Cu) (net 1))
 (segment (start 99.06 120.65) (end 99.06 118.745) (width 0.25) (layer F.Cu) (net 1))
 (segment (start 99.06 118.745) (end 99.06 114.3) (width 0.25) (layer F.Cu) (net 1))
 (segment (start 99.06 114.3) (end 99.52 113.84) (width 0.25) (layer F.Cu) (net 1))
 (segment (start 99.52 113.84) (end 100.33 113.84) (width 0.25) (layer F.Cu) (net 1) (status 800000)))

